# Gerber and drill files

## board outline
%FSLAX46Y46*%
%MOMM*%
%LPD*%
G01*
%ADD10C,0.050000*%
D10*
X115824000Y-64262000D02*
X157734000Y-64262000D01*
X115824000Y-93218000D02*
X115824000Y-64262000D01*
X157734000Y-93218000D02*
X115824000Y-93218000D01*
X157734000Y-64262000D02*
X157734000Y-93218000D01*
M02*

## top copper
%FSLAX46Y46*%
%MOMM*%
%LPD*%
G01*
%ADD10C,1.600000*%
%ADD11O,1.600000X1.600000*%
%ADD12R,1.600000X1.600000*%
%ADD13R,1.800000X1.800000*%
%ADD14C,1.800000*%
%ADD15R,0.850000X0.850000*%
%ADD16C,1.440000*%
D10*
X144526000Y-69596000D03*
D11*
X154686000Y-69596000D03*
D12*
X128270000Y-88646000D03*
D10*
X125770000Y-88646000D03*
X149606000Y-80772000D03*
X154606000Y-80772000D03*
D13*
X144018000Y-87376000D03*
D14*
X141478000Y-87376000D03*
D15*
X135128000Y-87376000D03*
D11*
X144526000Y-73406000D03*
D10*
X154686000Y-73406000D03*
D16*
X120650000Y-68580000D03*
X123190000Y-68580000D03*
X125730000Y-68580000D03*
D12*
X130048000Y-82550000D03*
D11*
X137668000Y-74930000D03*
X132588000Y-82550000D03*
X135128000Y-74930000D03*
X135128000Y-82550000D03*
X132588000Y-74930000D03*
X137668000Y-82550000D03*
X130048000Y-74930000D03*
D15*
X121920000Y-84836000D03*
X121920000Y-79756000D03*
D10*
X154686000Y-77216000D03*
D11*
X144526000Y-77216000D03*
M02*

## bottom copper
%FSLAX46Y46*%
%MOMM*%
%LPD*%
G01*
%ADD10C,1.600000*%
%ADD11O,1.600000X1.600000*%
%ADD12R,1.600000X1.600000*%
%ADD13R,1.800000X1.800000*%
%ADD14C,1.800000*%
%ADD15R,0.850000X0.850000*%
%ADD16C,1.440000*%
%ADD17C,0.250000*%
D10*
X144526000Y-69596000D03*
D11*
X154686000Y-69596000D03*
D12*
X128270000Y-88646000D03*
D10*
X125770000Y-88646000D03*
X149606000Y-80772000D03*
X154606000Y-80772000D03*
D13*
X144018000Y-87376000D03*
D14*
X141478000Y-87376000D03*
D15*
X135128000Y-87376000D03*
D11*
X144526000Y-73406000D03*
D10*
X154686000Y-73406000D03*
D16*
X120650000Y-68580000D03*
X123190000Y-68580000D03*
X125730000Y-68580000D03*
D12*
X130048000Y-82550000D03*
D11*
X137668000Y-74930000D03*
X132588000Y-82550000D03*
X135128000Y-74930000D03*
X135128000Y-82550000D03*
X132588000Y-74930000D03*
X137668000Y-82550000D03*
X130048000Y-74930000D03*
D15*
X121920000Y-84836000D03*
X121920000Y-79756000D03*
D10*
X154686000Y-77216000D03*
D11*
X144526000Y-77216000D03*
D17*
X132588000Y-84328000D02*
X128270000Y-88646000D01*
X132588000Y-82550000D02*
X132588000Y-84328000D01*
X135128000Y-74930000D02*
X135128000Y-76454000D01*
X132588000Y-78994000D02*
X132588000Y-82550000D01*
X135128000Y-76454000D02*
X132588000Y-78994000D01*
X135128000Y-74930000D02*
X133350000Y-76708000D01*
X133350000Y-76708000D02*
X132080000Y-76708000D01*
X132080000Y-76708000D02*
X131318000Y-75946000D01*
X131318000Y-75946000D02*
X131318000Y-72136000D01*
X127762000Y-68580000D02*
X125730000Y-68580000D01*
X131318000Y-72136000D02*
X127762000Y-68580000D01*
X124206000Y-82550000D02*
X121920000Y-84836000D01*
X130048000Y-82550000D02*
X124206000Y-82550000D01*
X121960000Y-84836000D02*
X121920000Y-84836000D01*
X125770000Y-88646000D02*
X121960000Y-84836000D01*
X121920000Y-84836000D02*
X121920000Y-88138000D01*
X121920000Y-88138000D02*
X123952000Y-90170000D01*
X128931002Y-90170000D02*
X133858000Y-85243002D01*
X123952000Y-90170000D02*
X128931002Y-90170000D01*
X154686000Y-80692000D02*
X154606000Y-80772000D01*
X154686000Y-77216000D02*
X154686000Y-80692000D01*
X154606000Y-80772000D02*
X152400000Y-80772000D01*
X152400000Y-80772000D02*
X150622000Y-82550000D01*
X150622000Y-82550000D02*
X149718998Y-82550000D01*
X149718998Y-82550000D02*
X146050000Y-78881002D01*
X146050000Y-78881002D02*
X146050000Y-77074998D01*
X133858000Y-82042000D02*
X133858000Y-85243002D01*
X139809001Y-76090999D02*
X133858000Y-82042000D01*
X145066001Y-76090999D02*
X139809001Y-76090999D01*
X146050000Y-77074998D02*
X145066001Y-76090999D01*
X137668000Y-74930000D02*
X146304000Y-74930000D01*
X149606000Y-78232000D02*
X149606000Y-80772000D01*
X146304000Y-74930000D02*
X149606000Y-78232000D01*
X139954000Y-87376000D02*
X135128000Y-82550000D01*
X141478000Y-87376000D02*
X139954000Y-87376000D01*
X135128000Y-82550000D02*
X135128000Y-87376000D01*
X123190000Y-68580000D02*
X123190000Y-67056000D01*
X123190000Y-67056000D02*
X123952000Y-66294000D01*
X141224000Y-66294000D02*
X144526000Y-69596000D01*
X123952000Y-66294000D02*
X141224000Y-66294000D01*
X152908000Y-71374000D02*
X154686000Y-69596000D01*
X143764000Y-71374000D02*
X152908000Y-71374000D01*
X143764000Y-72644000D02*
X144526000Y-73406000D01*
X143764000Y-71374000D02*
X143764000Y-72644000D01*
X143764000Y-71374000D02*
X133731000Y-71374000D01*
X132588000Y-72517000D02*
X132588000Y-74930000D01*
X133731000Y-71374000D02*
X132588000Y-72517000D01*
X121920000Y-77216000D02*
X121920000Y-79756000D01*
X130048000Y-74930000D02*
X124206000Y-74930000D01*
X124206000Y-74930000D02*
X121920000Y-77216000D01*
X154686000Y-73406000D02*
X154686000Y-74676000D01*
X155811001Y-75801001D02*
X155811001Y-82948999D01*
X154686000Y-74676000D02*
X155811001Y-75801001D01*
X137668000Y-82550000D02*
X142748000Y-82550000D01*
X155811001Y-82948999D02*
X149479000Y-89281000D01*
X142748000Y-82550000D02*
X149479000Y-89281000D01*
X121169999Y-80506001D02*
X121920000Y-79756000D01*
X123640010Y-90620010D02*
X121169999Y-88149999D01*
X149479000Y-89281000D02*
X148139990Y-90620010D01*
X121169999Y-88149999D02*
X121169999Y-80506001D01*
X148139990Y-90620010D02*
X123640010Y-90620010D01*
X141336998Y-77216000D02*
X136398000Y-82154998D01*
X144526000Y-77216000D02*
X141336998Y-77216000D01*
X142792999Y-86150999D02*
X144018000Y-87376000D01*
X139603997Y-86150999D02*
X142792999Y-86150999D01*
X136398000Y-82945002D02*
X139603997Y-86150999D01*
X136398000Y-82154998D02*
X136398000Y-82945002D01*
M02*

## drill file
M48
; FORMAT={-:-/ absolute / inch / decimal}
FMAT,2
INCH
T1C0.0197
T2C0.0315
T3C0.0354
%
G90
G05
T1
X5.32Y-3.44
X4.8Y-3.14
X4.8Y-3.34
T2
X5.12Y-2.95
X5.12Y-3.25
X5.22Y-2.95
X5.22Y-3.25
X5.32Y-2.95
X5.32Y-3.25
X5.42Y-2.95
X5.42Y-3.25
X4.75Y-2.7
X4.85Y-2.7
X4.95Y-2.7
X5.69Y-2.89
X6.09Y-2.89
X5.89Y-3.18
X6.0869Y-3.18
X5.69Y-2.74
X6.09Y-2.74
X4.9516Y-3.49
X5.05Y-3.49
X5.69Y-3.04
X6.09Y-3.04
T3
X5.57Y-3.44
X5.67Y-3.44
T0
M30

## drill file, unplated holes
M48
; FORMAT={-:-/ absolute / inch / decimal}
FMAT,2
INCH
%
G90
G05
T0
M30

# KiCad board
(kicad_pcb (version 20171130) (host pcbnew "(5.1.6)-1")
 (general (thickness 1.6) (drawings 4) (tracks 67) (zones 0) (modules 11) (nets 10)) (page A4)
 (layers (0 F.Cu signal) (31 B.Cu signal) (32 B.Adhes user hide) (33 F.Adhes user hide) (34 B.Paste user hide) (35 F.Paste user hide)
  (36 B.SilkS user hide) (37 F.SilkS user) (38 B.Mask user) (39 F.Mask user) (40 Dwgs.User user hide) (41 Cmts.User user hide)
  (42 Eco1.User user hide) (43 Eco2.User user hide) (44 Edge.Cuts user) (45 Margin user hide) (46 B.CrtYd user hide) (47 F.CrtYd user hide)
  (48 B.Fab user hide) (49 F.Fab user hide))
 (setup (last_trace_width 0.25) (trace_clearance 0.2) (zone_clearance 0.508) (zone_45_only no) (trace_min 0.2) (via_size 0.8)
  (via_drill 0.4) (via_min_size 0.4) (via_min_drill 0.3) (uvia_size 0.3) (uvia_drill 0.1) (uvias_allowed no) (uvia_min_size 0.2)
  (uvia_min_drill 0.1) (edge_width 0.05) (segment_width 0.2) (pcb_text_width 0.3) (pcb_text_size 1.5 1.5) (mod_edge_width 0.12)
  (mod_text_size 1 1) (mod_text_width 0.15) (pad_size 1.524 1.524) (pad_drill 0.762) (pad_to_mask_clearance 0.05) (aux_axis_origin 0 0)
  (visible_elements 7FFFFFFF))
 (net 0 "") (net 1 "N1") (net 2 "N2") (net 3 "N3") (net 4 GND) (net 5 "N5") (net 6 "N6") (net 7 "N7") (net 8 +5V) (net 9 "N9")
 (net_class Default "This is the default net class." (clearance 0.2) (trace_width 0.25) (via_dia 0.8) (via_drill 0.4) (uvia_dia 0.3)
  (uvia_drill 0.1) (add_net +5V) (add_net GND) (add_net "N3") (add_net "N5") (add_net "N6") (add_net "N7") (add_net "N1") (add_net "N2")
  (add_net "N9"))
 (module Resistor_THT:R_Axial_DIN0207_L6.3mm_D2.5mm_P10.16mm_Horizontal (layer F.Cu) (at 144.526 69.596)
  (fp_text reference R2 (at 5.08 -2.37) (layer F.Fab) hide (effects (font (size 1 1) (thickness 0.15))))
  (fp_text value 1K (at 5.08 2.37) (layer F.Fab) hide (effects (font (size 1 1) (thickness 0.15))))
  (pad 1 thru_hole circle (at 0 0) (size 1.6 1.6) (drill 0.8) (layers *.Cu *.Mask) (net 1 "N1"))
  (pad 2 thru_hole oval (at 10.16 0) (size 1.6 1.6) (drill 0.8) (layers *.Cu *.Mask) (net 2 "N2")))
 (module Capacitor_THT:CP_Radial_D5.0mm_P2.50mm (layer F.Cu) (at 128.27 88.646 180)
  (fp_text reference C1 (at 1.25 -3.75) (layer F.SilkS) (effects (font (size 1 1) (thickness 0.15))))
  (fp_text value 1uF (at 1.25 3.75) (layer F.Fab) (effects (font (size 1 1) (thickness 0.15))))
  (pad 1 thru_hole rect (at 0 0 180) (size 1.6 1.6) (drill 0.8) (layers *.Cu *.Mask) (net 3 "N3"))
  (pad 2 thru_hole circle (at 2.5 0 180) (size 1.6 1.6) (drill 0.8) (layers *.Cu *.Mask) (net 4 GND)))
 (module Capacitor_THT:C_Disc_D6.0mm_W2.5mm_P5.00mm (layer F.Cu) (at 149.606 80.772)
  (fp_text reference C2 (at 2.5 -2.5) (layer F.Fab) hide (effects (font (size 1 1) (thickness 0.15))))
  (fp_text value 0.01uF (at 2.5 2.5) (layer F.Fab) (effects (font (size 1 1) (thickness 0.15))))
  (pad 1 thru_hole circle (at 0 0) (size 1.6 1.6) (drill 0.8) (layers *.Cu *.Mask) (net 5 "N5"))
  (pad 2 thru_hole circle (at 5 0) (size 1.6 1.6) (drill 0.8) (layers *.Cu *.Mask) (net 4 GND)))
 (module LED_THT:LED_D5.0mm (layer F.Cu) (at 144.018 87.376 180)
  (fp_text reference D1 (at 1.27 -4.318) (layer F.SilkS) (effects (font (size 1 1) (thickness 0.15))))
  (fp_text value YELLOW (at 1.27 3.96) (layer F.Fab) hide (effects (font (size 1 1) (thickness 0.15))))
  (pad 1 thru_hole rect (at 0 0 180) (size 1.8 1.8) (drill 0.9) (layers *.Cu *.Mask) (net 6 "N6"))
  (pad 2 thru_hole circle (at 2.54 0 180) (size 1.8 1.8) (drill 0.9) (layers *.Cu *.Mask) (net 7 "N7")))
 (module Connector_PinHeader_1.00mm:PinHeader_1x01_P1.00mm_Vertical (layer F.Cu) (at 135.128 87.376)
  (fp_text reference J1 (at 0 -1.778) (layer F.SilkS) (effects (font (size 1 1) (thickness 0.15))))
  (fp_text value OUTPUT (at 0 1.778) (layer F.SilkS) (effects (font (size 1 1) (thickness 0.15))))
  (pad 1 thru_hole rect (at 0 0) (size 0.85 0.85) (drill 0.5) (layers *.Cu *.Mask) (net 7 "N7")))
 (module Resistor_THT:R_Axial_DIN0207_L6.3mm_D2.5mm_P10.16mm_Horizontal (layer F.Cu) (at 154.686 73.406 180)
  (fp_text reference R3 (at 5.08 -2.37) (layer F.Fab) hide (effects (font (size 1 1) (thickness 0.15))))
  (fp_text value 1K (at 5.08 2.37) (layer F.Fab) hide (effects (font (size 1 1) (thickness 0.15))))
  (pad 2 thru_hole oval (at 10.16 0 180) (size 1.6 1.6) (drill 0.8) (layers *.Cu *.Mask) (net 2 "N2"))
  (pad 1 thru_hole circle (at 0 0 180) (size 1.6 1.6) (drill 0.8) (layers *.Cu *.Mask) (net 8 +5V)))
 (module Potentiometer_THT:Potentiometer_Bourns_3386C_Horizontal (layer F.Cu) (at 125.73 68.58 270)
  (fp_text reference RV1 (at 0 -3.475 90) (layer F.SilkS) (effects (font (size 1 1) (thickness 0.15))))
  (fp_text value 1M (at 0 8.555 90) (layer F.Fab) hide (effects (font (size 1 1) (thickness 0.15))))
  (pad 3 thru_hole circle (at 0 5.08 270) (size 1.44 1.44) (drill 0.8) (layers *.Cu *.Mask) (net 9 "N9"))
  (pad 2 thru_hole circle (at 0 2.54 270) (size 1.44 1.44) (drill 0.8) (layers *.Cu *.Mask) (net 1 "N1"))
  (pad 1 thru_hole circle (at 0 0 270) (size 1.44 1.44) (drill 0.8) (layers *.Cu *.Mask) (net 3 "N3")))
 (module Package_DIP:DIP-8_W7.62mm (layer F.Cu) (at 130.048 82.55 90)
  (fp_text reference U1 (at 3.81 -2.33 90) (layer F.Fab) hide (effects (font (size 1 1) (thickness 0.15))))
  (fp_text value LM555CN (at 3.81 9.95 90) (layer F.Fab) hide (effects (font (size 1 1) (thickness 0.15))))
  (pad 1 thru_hole rect (at 0 0 90) (size 1.6 1.6) (drill 0.8) (layers *.Cu *.Mask) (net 4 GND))
  (pad 5 thru_hole oval (at 7.62 7.62 90) (size 1.6 1.6) (drill 0.8) (layers *.Cu *.Mask) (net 5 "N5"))
  (pad 2 thru_hole oval (at 0 2.54 90) (size 1.6 1.6) (drill 0.8) (layers *.Cu *.Mask) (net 3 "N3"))
  (pad 6 thru_hole oval (at 7.62 5.08 90) (size 1.6 1.6) (drill 0.8) (layers *.Cu *.Mask) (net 3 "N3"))
  (pad 3 thru_hole oval (at 0 5.08 90) (size 1.6 1.6) (drill 0.8) (layers *.Cu *.Mask) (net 7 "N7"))
  (pad 7 thru_hole oval (at 7.62 2.54 90) (size 1.6 1.6) (drill 0.8) (layers *.Cu *.Mask) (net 2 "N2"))
  (pad 4 thru_hole oval (at 0 7.62 90) (size 1.6 1.6) (drill 0.8) (layers *.Cu *.Mask) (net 8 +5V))
  (pad 8 thru_hole oval (at 7.62 0 90) (size 1.6 1.6) (drill 0.8) (layers *.Cu *.Mask) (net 8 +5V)))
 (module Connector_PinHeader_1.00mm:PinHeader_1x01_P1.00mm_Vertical (layer F.Cu) (at 121.92 84.836)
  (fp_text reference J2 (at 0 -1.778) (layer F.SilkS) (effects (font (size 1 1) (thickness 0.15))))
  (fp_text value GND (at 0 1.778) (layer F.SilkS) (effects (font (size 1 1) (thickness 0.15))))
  (pad 1 thru_hole rect (at 0 0) (size 0.85 0.85) (drill 0.5) (layers *.Cu *.Mask) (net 4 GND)))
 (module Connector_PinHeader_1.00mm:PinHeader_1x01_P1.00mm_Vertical (layer F.Cu) (at 121.92 79.756)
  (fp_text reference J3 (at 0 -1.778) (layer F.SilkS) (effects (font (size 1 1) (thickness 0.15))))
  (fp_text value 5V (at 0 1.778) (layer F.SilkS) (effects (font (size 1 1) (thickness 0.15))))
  (pad 1 thru_hole rect (at 0 0) (size 0.85 0.85) (drill 0.5) (layers *.Cu *.Mask) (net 8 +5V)))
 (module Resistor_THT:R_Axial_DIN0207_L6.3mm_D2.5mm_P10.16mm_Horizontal (layer F.Cu) (at 154.686 77.216 180)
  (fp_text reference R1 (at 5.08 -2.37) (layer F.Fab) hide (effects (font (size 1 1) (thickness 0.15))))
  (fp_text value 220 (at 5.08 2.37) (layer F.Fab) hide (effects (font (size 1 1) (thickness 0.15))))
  (pad 1 thru_hole circle (at 0 0 180) (size 1.6 1.6) (drill 0.8) (layers *.Cu *.Mask) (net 4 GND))
  (pad 2 thru_hole oval (at 10.16 0 180) (size 1.6 1.6) (drill 0.8) (layers *.Cu *.Mask) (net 6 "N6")))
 (gr_line (start 115.824 64.262) (end 157.734 64.262) (layer Edge.Cuts) (width 0.05))
 (gr_line (start 115.824 93.218) (end 115.824 64.262) (layer Edge.Cuts) (width 0.05))
 (gr_line (start 157.734 93.218) (end 115.824 93.218) (layer Edge.Cuts) (width 0.05))
 (gr_line (start 157.734 64.262) (end 157.734 93.218) (layer Edge.Cuts) (width 0.05))
 (segment (start 132.588 84.328) (end 128.27 88.646) (width 0.25) (layer B.Cu) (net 3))
 (segment (start 132.588 82.55) (end 132.588 84.328) (width 0.25) (layer B.Cu) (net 3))
 (segment (start 135.128 74.93) (end 135.128 76.454) (width 0.25) (layer B.Cu) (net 3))
 (segment (start 132.588 78.994) (end 132.588 82.55) (width 0.25) (layer B.Cu) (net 3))
 (segment (start 135.128 76.454) (end 132.588 78.994) (width 0.25) (layer B.Cu) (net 3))
 (segment (start 135.128 74.93) (end 133.35 76.708) (width 0.25) (layer B.Cu) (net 3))
 (segment (start 133.35 76.708) (end 132.08 76.708) (width 0.25) (layer B.Cu) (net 3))
 (segment (start 132.08 76.708) (end 131.318 75.946) (width 0.25) (layer B.Cu) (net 3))
 (segment (start 131.318 75.946) (end 131.318 72.136) (width 0.25) (layer B.Cu) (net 3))
 (segment (start 127.762 68.58) (end 125.73 68.58) (width 0.25) (layer B.Cu) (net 3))
 (segment (start 131.318 72.136) (end 127.762 68.58) (width 0.25) (layer B.Cu) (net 3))
 (segment (start 124.206 82.55) (end 121.92 84.836) (width 0.25) (layer B.Cu) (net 4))
 (segment (start 130.048 82.55) (end 124.206 82.55) (width 0.25) (layer B.Cu) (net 4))
 (segment (start 121.96 84.836) (end 121.92 84.836) (width 0.25) (layer B.Cu) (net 4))
 (segment (start 125.77 88.646) (end 121.96 84.836) (width 0.25) (layer B.Cu) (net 4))
 (segment (start 121.92 84.836) (end 121.92 88.138) (width 0.25) (layer B.Cu) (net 4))
 (segment (start 121.92 88.138) (end 123.952 90.17) (width 0.25) (layer B.Cu) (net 4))
 (segment (start 128.931002 90.17) (end 133.858 85.243002) (width 0.25) (layer B.Cu) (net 4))
 (segment (start 123.952 90.17) (end 128.931002 90.17) (width 0.25) (layer B.Cu) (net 4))
 (segment (start 154.686 80.692) (end 154.606 80.772) (width 0.25) (layer B.Cu) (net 4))
 (segment (start 154.686 77.216) (end 154.686 80.692) (width 0.25) (layer B.Cu) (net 4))
 (segment (start 154.606 80.772) (end 152.4 80.772) (width 0.25) (layer B.Cu) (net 4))
 (segment (start 152.4 80.772) (end 150.622 82.55) (width 0.25) (layer B.Cu) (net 4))
 (segment (start 150.622 82.55) (end 149.718998 82.55) (width 0.25) (layer B.Cu) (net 4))
 (segment (start 149.718998 82.55) (end 146.05 78.881002) (width 0.25) (layer B.Cu) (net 4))
 (segment (start 146.05 78.881002) (end 146.05 77.074998) (width 0.25) (layer B.Cu) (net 4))
 (segment (start 133.858 82.042) (end 133.858 85.243002) (width 0.25) (layer B.Cu) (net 4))
 (segment (start 139.809001 76.090999) (end 133.858 82.042) (width 0.25) (layer B.Cu) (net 4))
 (segment (start 145.066001 76.090999) (end 139.809001 76.090999) (width 0.25) (layer B.Cu) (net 4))
 (segment (start 146.05 77.074998) (end 145.066001 76.090999) (width 0.25) (layer B.Cu) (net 4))
 (segment (start 137.668 74.93) (end 146.304 74.93) (width 0.25) (layer B.Cu) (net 5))
 (segment (start 149.606 78.232) (end 149.606 80.772) (width 0.25) (layer B.Cu) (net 5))
 (segment (start 146.304 74.93) (end 149.606 78.232) (width 0.25) (layer B.Cu) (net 5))
 (segment (start 139.954 87.376) (end 135.128 82.55) (width 0.25) (layer B.Cu) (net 7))
 (segment (start 141.478 87.376) (end 139.954 87.376) (width 0.25) (layer B.Cu) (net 7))
 (segment (start 135.128 82.55) (end 135.128 87.376) (width 0.25) (layer B.Cu) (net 7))
 (segment (start 123.19 68.58) (end 123.19 67.056) (width 0.25) (layer B.Cu) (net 1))
 (segment (start 123.19 67.056) (end 123.952 66.294) (width 0.25) (layer B.Cu) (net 1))
 (segment (start 141.224 66.294) (end 144.526 69.596) (width 0.25) (layer B.Cu) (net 1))
 (segment (start 123.952 66.294) (end 141.224 66.294) (width 0.25) (layer B.Cu) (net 1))
 (segment (start 152.908 71.374) (end 154.686 69.596) (width 0.25) (layer B.Cu) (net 2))
 (segment (start 143.764 71.374) (end 152.908 71.374) (width 0.25) (layer B.Cu) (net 2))
 (segment (start 143.764 72.644) (end 144.526 73.406) (width 0.25) (layer B.Cu) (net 2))
 (segment (start 143.764 71.374) (end 143.764 72.644) (width 0.25) (layer B.Cu) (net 2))
 (segment (start 143.764 71.374) (end 133.731 71.374) (width 0.25) (layer B.Cu) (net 2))
 (segment (start 132.588 72.517) (end 132.588 74.93) (width 0.25) (layer B.Cu) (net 2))
 (segment (start 133.731 71.374) (end 132.588 72.517) (width 0.25) (layer B.Cu) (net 2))
 (segment (start 121.92 77.216) (end 121.92 79.756) (width 0.25) (layer B.Cu) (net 8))
 (segment (start 130.048 74.93) (end 124.206 74.93) (width 0.25) (layer B.Cu) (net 8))
 (segment (start 124.206 74.93) (end 121.92 77.216) (width 0.25) (layer B.Cu) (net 8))
 (segment (start 154.686 73.406) (end 154.686 74.676) (width 0.25) (layer B.Cu) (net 8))
 (segment (start 155.811001 75.801001) (end 155.811001 82.948999) (width 0.25) (layer B.Cu) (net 8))
 (segment (start 154.686 74.676) (end 155.811001 75.801001) (width 0.25) (layer B.Cu) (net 8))
 (segment (start 137.668 82.55) (end 142.748 82.55) (width 0.25) (layer B.Cu) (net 8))
 (segment (start 155.811001 82.948999) (end 149.479 89.281) (width 0.25) (layer B.Cu) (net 8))
 (segment (start 142.748 82.55) (end 149.479 89.281) (width 0.25) (layer B.Cu) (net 8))
 (segment (start 121.169999 80.506001) (end 121.92 79.756) (width 0.25) (layer B.Cu) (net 8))
 (segment (start 123.64001 90.62001) (end 121.169999 88.149999) (width 0.25) (layer B.Cu) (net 8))
 (segment (start 149.479 89.281) (end 148.13999 90.62001) (width 0.25) (layer B.Cu) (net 8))
 (segment (start 121.169999 88.149999) (end 121.169999 80.506001) (width 0.25) (layer B.Cu) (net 8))
 (segment (start 148.13999 90.62001) (end 123.64001 90.62001) (width 0.25) (layer B.Cu) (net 8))
 (segment (start 141.336998 77.216) (end 136.398 82.154998) (width 0.25) (layer B.Cu) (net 6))
 (segment (start 144.526 77.216) (end 141.336998 77.216) (width 0.25) (layer B.Cu) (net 6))
 (segment (start 142.792999 86.150999) (end 144.018 87.376) (width 0.25) (layer B.Cu) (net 6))
 (segment (start 139.603997 86.150999) (end 142.792999 86.150999) (width 0.25) (layer B.Cu) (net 6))
 (segment (start 136.398 82.945002) (end 139.603997 86.150999) (width 0.25) (layer B.Cu) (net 6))
 (segment (start 136.398 82.154998) (end 136.398 82.945002) (width 0.25) (layer B.Cu) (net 6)))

